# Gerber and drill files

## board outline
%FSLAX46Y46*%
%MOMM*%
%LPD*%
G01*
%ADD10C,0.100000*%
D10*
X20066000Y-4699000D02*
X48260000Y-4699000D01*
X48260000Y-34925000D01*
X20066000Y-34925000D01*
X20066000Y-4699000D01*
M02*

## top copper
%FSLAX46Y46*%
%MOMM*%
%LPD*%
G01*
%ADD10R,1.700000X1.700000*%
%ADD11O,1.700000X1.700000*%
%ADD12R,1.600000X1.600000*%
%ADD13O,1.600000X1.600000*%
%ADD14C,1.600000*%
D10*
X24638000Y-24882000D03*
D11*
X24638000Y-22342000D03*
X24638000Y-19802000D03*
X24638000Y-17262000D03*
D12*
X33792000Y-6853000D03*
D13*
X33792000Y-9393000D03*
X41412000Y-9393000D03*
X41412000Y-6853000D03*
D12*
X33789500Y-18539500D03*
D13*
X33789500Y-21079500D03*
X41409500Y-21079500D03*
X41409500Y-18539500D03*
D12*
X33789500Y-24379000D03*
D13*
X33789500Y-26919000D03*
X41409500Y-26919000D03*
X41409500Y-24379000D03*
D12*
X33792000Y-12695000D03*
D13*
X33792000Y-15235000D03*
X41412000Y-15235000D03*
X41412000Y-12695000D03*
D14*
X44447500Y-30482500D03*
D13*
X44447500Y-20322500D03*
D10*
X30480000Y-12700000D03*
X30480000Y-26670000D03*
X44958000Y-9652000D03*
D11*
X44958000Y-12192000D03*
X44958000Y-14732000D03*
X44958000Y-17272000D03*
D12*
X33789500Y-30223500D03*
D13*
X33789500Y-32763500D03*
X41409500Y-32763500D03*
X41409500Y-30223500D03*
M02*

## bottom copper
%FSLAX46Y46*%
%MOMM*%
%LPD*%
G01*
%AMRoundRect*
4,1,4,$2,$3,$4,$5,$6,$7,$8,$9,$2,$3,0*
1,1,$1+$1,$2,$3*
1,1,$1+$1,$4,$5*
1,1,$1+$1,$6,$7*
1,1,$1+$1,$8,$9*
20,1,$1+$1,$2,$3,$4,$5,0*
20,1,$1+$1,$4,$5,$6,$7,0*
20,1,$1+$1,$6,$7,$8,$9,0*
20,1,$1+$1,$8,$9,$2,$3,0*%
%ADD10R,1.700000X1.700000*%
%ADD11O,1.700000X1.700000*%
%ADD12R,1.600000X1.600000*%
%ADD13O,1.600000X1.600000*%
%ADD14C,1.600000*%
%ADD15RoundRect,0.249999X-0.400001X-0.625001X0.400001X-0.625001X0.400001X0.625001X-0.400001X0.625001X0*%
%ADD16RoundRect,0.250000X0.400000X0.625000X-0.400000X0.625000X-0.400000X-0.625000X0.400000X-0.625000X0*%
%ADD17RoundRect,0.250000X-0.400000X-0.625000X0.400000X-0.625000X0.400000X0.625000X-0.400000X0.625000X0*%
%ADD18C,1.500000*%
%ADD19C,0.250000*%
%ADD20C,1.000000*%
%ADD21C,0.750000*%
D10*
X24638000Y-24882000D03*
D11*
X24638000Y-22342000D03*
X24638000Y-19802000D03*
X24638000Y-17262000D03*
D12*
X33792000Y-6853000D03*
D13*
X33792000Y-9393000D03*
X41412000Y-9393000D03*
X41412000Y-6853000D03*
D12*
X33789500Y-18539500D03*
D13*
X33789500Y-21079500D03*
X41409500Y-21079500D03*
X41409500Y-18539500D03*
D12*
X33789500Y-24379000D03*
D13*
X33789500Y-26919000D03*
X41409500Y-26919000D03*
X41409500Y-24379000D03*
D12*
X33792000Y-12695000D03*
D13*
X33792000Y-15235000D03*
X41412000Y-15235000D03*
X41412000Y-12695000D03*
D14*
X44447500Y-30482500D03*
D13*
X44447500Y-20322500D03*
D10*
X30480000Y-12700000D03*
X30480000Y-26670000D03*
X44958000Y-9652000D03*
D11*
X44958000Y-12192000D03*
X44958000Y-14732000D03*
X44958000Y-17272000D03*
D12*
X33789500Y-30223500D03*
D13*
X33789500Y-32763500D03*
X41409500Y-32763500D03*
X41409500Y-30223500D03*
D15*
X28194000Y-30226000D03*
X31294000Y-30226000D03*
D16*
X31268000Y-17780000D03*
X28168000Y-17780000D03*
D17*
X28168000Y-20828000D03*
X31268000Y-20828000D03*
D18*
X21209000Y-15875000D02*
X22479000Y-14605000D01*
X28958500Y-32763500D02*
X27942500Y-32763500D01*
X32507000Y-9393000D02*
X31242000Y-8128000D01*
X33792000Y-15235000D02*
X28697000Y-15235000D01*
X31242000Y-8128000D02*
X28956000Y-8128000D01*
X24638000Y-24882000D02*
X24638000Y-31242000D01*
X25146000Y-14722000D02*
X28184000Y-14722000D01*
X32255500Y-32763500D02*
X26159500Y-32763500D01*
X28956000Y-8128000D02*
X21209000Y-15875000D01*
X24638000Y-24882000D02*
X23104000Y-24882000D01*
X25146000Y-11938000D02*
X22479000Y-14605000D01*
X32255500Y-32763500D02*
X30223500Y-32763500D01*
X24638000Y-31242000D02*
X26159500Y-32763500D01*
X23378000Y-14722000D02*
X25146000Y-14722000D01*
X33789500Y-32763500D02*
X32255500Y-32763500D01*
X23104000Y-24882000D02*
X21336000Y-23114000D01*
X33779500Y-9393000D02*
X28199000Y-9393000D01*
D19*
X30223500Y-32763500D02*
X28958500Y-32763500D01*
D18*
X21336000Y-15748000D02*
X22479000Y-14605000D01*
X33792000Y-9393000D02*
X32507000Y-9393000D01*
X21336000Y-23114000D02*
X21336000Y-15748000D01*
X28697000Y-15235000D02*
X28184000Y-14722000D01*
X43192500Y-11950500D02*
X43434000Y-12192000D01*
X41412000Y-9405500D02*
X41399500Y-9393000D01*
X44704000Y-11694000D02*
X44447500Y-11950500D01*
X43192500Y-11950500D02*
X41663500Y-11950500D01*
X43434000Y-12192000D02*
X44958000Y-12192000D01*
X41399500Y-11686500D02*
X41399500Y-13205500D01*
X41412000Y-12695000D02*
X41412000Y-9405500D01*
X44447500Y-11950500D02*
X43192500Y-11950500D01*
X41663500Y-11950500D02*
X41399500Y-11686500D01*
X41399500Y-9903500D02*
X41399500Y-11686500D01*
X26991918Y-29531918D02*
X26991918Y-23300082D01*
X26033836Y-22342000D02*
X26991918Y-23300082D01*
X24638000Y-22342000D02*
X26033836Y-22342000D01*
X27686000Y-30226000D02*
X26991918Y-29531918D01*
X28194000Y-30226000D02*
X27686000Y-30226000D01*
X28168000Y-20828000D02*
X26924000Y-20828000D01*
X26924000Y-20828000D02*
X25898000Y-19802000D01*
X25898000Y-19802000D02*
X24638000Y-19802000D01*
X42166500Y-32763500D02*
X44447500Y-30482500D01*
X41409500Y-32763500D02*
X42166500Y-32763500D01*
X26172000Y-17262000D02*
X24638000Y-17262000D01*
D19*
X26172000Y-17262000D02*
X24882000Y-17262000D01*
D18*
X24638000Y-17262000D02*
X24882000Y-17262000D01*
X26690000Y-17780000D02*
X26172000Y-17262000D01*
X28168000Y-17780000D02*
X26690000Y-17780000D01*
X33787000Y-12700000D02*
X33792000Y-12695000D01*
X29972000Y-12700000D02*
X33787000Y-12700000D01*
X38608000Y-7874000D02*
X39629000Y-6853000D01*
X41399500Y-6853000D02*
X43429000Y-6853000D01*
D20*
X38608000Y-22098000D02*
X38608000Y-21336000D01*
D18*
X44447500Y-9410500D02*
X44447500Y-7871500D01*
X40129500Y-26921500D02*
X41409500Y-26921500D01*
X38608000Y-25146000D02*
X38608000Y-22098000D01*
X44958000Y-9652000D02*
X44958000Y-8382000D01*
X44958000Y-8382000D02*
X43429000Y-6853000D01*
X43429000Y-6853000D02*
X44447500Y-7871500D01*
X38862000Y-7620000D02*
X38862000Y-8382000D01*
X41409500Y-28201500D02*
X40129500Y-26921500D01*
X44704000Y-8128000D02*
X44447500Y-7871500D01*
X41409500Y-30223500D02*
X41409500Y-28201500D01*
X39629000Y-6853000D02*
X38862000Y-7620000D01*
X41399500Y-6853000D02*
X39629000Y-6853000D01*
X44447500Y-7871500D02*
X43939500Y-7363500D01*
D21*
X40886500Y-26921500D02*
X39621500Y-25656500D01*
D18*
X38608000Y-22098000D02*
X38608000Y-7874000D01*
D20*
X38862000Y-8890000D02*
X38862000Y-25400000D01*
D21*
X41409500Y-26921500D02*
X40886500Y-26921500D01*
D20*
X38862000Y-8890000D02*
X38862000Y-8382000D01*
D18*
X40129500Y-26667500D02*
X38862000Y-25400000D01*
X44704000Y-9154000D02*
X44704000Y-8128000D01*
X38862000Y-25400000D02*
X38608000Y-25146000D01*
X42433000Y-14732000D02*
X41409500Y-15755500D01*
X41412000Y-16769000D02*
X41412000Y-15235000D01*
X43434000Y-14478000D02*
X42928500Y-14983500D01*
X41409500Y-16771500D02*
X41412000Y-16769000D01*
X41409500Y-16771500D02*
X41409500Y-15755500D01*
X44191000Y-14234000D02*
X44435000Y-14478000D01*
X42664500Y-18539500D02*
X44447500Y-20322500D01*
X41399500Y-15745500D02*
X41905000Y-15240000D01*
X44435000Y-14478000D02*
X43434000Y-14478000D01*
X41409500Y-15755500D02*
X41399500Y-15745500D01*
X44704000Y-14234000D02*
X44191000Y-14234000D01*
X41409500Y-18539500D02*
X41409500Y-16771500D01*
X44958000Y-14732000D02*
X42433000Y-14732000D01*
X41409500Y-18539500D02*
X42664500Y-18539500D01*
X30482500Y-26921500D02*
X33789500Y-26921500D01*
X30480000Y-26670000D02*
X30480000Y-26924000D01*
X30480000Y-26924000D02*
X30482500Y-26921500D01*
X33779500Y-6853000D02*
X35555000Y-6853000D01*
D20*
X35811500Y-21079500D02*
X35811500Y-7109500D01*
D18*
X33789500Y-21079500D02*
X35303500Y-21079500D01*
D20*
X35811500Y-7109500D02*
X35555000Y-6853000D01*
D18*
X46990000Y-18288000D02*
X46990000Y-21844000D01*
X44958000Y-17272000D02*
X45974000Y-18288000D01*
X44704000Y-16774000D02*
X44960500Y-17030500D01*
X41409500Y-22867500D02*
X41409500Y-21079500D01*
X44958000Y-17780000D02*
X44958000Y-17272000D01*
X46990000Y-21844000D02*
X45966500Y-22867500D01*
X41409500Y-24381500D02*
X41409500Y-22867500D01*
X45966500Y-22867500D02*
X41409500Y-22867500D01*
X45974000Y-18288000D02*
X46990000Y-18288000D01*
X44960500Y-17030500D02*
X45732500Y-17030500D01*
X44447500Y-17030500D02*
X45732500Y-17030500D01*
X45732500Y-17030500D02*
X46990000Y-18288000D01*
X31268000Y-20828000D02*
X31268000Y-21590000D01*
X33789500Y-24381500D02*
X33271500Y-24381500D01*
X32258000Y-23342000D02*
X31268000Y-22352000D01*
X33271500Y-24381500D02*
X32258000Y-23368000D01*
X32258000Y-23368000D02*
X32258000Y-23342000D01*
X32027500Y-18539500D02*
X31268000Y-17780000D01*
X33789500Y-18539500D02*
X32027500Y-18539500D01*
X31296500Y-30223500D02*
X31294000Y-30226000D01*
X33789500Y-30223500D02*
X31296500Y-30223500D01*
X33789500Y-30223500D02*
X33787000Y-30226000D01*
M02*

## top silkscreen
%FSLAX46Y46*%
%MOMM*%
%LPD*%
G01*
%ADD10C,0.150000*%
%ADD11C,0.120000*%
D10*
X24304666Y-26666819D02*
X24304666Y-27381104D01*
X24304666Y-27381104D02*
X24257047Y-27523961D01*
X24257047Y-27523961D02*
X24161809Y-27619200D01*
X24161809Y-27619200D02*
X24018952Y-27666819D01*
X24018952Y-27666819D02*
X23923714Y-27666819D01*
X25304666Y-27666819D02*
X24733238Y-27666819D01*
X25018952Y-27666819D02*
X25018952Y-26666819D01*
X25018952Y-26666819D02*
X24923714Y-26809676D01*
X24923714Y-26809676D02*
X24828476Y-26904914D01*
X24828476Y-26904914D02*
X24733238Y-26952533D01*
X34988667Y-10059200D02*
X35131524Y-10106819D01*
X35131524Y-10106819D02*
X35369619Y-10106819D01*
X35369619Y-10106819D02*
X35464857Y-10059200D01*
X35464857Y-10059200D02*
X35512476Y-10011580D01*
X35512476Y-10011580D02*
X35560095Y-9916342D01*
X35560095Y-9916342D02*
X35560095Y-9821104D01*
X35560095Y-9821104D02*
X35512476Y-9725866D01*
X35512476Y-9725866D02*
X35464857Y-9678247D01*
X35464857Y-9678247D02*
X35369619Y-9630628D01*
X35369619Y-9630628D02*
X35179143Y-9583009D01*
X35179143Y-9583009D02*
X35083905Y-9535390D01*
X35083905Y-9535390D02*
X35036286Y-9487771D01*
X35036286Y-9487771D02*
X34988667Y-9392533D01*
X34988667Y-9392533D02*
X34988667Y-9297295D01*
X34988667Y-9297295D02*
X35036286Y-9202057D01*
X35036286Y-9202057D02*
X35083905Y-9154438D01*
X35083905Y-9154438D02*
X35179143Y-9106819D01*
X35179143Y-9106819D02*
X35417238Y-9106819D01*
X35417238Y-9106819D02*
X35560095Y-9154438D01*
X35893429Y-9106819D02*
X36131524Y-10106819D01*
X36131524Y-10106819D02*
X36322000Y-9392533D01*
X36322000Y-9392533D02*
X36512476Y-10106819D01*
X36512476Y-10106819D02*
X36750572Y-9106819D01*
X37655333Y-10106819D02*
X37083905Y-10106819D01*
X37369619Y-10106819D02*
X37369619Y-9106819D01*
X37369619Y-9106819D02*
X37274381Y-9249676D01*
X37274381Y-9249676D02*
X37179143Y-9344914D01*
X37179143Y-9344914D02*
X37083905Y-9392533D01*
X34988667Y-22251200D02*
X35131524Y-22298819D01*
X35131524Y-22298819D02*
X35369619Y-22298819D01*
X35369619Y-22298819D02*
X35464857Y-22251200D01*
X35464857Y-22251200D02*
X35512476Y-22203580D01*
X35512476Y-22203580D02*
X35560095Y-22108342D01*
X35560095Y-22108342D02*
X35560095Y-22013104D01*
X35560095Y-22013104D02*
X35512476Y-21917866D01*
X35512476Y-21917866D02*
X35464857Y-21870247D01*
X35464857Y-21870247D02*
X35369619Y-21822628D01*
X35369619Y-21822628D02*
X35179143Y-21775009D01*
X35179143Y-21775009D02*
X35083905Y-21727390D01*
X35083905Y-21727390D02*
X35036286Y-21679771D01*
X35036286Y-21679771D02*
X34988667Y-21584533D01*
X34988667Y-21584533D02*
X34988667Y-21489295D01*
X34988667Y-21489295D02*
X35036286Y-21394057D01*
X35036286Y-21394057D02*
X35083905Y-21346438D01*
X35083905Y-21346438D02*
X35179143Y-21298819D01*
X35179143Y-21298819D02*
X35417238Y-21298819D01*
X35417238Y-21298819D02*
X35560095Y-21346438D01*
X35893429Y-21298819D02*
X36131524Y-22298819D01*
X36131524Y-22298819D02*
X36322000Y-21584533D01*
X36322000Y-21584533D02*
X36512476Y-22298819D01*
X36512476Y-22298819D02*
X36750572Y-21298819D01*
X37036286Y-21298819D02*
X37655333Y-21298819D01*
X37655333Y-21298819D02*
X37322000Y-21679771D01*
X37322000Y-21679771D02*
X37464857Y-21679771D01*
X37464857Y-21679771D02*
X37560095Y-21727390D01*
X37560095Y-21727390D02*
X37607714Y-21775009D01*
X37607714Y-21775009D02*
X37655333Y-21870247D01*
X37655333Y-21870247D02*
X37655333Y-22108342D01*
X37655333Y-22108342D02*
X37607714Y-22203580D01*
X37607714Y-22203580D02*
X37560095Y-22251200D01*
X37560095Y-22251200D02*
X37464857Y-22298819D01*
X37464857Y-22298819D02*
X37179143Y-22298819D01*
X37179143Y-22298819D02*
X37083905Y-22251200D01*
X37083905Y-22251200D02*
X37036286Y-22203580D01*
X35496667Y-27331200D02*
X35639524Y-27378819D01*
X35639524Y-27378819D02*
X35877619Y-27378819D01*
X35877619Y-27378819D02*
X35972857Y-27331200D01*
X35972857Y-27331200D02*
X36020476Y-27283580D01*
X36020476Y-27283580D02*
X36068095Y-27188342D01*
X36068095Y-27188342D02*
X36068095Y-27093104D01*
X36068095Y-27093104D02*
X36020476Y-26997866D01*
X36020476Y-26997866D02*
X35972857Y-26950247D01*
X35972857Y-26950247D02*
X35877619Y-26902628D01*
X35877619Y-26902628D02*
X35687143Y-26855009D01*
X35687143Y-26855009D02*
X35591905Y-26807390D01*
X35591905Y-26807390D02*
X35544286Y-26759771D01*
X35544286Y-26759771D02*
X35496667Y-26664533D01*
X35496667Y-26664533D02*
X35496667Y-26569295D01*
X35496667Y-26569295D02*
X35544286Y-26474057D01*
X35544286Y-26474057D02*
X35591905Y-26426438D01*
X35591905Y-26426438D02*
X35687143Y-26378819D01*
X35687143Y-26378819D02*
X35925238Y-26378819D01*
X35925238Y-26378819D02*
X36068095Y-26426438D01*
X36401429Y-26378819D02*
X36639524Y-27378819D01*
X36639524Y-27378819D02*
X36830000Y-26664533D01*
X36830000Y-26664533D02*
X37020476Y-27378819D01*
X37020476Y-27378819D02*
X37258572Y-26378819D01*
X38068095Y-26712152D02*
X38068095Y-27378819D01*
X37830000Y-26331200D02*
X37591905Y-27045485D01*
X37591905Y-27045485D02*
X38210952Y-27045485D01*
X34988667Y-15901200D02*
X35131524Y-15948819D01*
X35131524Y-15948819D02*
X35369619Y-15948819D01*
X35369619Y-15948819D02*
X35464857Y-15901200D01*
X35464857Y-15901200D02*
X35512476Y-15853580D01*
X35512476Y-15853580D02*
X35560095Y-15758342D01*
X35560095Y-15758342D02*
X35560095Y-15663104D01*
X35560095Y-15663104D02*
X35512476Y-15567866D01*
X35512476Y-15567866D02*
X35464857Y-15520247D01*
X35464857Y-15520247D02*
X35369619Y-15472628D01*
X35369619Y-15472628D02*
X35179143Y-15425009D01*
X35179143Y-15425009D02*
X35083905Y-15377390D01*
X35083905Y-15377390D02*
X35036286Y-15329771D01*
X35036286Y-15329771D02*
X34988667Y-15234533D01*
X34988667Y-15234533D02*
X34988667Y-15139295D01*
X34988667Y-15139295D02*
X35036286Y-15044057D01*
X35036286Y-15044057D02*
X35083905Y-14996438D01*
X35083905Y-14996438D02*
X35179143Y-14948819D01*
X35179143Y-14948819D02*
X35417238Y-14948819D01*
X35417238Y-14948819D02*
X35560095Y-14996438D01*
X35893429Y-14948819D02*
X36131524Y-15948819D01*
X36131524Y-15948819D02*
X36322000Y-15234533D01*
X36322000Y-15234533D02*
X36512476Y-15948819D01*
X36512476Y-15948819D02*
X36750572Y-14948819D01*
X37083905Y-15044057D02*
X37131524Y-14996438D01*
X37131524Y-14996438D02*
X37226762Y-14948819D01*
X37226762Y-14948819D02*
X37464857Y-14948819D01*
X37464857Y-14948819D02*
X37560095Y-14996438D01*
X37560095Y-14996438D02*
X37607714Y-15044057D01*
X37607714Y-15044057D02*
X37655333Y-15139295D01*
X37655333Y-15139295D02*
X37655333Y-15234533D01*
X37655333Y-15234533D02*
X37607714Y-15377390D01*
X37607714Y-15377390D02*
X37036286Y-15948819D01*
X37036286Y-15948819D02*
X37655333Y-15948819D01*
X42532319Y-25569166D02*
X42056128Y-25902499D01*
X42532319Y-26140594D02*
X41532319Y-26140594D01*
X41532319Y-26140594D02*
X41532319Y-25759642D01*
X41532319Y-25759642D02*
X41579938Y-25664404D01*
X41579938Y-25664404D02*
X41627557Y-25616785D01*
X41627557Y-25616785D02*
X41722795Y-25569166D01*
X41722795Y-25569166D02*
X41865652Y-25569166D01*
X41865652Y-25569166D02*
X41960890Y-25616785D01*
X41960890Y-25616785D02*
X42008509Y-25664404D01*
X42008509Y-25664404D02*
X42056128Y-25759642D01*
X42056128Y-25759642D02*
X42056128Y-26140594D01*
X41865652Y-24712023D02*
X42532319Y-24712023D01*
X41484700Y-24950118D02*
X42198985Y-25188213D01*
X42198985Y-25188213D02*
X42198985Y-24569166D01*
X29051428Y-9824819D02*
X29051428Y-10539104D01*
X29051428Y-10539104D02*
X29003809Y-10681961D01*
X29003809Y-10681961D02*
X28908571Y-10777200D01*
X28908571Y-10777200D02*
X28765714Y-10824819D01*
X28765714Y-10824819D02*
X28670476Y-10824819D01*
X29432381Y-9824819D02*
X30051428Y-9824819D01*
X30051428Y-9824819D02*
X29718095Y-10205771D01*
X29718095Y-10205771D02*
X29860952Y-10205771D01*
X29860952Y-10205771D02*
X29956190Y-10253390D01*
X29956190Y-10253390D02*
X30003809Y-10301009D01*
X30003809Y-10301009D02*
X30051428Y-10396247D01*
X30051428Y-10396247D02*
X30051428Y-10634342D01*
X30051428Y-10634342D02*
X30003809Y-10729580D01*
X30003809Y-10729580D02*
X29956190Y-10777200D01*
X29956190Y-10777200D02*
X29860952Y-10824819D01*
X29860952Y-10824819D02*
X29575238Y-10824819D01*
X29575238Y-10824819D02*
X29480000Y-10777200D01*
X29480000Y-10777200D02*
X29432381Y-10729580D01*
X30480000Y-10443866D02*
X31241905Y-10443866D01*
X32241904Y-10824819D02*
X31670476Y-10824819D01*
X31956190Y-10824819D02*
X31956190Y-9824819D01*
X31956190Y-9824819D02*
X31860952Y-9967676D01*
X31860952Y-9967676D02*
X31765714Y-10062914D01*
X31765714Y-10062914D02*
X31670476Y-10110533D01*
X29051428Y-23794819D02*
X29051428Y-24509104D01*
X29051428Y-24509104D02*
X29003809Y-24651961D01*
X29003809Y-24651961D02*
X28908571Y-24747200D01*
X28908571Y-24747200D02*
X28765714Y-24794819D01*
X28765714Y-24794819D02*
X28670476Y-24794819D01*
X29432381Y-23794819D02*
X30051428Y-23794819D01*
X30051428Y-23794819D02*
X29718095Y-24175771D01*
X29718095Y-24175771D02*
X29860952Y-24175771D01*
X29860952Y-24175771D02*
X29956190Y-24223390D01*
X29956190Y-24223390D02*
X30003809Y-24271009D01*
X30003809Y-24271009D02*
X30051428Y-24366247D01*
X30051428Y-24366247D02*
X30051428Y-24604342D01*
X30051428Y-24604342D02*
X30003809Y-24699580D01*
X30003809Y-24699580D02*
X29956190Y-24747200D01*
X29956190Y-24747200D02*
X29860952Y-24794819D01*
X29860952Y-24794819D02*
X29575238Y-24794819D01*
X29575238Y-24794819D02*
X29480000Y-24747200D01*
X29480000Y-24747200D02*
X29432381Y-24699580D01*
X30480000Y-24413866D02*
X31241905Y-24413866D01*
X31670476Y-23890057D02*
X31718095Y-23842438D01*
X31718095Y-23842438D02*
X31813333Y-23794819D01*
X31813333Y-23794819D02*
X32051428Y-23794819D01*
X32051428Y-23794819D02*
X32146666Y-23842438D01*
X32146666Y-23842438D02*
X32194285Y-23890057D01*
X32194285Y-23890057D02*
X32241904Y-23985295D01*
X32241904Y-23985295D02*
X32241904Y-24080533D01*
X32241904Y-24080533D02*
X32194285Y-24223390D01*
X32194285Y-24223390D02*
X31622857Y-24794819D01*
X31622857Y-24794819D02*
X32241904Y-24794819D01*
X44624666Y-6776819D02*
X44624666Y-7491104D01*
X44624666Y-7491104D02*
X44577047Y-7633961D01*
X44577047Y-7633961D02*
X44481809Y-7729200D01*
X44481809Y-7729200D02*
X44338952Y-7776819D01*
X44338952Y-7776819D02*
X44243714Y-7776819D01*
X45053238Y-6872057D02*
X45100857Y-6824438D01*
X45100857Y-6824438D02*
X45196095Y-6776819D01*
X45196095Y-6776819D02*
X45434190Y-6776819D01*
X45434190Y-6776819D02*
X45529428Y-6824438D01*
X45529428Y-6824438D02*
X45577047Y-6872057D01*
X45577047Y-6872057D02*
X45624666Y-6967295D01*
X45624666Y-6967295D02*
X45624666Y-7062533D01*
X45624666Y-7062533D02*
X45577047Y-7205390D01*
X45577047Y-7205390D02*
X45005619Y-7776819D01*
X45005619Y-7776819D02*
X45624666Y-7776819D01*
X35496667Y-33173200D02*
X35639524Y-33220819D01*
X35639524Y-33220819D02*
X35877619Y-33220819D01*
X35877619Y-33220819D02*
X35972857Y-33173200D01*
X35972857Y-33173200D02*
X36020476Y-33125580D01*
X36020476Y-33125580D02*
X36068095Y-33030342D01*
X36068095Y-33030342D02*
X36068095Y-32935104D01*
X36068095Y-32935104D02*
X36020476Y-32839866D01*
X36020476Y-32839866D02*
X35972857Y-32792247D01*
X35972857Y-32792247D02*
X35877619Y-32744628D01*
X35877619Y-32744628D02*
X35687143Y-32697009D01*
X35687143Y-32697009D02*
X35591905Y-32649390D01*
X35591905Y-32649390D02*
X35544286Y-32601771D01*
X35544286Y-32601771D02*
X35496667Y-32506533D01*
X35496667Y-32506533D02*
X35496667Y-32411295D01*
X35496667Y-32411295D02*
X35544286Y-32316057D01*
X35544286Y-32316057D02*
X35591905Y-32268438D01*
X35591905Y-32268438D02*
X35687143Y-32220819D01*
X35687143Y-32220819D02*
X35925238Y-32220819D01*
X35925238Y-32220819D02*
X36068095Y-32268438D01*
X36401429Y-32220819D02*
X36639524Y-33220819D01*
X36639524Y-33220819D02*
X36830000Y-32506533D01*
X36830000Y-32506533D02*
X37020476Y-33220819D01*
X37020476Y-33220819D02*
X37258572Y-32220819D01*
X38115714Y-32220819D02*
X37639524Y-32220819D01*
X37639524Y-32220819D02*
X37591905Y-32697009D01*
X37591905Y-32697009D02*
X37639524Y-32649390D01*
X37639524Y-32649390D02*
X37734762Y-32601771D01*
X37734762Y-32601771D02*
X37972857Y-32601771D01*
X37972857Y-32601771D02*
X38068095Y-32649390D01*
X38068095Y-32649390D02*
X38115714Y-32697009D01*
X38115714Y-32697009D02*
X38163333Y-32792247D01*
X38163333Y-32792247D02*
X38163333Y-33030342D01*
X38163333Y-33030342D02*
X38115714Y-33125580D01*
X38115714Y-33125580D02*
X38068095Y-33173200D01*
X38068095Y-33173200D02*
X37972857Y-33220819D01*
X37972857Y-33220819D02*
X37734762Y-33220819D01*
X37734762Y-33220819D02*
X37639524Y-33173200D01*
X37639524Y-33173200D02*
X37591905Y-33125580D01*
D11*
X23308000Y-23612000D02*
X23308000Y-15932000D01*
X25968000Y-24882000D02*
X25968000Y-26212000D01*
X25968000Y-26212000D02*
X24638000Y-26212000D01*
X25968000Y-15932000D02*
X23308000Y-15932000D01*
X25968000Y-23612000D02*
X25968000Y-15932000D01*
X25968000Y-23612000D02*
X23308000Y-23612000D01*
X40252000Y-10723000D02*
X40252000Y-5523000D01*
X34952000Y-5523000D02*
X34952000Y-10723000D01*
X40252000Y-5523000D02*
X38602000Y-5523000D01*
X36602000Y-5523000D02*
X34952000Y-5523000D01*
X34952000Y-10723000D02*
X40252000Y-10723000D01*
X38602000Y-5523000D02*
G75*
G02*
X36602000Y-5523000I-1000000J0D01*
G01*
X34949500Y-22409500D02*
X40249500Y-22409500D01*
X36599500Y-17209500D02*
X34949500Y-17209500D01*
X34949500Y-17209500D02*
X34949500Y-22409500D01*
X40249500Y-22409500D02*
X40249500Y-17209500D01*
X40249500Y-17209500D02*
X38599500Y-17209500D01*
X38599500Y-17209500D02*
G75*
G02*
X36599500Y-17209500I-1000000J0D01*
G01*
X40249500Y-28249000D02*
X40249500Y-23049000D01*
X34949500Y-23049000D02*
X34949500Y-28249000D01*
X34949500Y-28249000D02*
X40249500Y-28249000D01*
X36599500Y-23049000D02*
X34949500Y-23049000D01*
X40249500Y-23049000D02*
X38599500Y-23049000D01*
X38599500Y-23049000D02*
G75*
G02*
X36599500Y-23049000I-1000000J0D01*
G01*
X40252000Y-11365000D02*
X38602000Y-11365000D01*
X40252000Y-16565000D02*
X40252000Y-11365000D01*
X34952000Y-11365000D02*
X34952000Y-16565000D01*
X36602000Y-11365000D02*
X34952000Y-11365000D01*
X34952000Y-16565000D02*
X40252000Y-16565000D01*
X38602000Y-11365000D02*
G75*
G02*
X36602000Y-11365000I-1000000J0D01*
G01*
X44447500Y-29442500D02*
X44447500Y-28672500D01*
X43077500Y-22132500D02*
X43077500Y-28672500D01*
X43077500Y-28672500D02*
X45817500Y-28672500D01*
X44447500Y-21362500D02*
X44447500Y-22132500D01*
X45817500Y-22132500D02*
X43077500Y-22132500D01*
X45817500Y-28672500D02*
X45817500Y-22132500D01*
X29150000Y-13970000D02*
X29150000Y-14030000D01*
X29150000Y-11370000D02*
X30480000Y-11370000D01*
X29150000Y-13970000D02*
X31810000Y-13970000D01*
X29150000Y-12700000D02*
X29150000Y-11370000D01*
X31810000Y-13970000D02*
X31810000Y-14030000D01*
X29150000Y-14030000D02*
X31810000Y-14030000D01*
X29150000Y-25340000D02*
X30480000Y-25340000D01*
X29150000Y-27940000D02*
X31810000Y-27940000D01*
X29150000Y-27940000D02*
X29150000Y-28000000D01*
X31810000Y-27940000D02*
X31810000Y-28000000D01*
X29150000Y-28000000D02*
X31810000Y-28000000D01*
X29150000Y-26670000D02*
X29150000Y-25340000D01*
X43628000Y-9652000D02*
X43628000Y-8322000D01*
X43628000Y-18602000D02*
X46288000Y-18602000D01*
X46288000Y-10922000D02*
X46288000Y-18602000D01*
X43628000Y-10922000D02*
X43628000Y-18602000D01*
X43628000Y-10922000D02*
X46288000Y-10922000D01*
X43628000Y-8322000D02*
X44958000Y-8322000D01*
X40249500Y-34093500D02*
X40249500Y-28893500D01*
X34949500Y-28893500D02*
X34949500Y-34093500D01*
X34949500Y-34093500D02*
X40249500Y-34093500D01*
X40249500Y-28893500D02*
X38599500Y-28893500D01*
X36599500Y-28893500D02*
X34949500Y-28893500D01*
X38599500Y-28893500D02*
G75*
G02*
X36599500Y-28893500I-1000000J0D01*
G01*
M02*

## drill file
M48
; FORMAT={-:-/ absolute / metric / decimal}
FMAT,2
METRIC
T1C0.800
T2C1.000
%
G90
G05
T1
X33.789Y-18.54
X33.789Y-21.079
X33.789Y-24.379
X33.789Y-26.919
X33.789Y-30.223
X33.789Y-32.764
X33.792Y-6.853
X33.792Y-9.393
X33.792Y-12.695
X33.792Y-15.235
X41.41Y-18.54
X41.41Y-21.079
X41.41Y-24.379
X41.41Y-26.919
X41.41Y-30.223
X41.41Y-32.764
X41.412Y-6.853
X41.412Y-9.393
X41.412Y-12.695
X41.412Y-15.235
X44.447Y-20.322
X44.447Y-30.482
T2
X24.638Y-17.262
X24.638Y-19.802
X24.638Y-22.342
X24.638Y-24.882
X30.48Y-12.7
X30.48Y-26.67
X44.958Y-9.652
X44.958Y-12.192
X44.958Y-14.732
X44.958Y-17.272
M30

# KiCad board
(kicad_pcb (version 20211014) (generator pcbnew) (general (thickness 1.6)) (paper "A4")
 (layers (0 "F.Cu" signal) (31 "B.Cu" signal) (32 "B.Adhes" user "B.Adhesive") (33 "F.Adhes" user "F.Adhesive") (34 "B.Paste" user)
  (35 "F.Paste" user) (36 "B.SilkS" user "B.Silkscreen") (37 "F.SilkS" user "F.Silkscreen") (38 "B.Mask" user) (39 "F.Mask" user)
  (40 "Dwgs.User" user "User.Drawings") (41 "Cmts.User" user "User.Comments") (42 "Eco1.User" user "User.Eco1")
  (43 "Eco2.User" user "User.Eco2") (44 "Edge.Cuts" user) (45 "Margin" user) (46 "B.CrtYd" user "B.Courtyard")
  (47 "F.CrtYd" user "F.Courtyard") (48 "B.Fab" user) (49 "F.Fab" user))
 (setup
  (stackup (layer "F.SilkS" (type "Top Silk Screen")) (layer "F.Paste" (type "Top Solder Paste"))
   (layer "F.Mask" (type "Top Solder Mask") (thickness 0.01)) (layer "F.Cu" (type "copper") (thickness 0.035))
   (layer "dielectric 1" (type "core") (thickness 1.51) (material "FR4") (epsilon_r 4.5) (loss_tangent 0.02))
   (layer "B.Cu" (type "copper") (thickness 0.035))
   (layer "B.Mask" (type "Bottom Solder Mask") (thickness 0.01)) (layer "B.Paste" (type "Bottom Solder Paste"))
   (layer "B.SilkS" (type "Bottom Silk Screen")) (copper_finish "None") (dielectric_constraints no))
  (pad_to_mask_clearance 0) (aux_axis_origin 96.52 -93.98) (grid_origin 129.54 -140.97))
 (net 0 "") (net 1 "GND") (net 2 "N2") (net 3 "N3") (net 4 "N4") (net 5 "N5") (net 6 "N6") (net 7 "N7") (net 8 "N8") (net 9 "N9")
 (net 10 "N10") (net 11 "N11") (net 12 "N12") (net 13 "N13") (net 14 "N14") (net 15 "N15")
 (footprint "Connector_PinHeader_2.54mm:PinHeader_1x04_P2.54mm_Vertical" (layer "F.Cu") (at 24.638 24.882 180)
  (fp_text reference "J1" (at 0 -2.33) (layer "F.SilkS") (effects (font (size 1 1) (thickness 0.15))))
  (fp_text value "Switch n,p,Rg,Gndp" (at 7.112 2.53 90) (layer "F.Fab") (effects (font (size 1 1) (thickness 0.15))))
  (fp_line (start 1.33 1.27) (end 1.33 8.95) (layer "F.SilkS") (width 0.12))
  (fp_line (start -1.33 0) (end -1.33 -1.33) (layer "F.SilkS") (width 0.12))
  (fp_line (start -1.33 -1.33) (end 0 -1.33) (layer "F.SilkS") (width 0.12))
  (fp_line (start -1.33 8.95) (end 1.33 8.95) (layer "F.SilkS") (width 0.12))
  (fp_line (start -1.33 1.27) (end -1.33 8.95) (layer "F.SilkS") (width 0.12))
  (fp_line (start -1.33 1.27) (end 1.33 1.27) (layer "F.SilkS") (width 0.12))
  (pad "1" thru_hole rect (at 0 0 180) (size 1.7 1.7) (drill 1) (layers *.Cu *.Mask) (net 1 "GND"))
  (pad "2" thru_hole oval (at 0 2.54 180) (size 1.7 1.7) (drill 1) (layers *.Cu *.Mask) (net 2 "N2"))
  (pad "3" thru_hole oval (at 0 5.08 180) (size 1.7 1.7) (drill 1) (layers *.Cu *.Mask) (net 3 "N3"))
  (pad "4" thru_hole oval (at 0 7.62 180) (size 1.7 1.7) (drill 1) (layers *.Cu *.Mask) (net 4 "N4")))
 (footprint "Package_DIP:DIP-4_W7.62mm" (layer "F.Cu") (at 33.792 6.853)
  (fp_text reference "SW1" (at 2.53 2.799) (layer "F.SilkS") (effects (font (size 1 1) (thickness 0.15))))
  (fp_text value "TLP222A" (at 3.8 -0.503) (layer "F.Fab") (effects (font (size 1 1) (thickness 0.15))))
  (fp_line (start 6.46 3.87) (end 6.46 -1.33) (layer "F.SilkS") (width 0.12))
  (fp_line (start 1.16 -1.33) (end 1.16 3.87) (layer "F.SilkS") (width 0.12))
  (fp_line (start 6.46 -1.33) (end 4.81 -1.33) (layer "F.SilkS") (width 0.12))
  (fp_line (start 2.81 -1.33) (end 1.16 -1.33) (layer "F.SilkS") (width 0.12))
  (fp_line (start 1.16 3.87) (end 6.46 3.87) (layer "F.SilkS") (width 0.12))
  (fp_arc (start 4.81 -1.33) (mid 3.81 -0.33) (end 2.81 -1.33) (layer "F.SilkS") (width 0.12))
  (pad "1" thru_hole rect locked (at 0 0) (size 1.6 1.6) (drill 0.8) (layers *.Cu *.Mask) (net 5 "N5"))
  (pad "2" thru_hole oval locked (at 0 2.54) (size 1.6 1.6) (drill 0.8) (layers *.Cu *.Mask) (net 1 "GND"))
  (pad "3" thru_hole oval locked (at 7.62 2.54) (size 1.6 1.6) (drill 0.8) (layers *.Cu *.Mask) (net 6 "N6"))
  (pad "4" thru_hole oval locked (at 7.62 0) (size 1.6 1.6) (drill 0.8) (layers *.Cu *.Mask) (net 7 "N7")))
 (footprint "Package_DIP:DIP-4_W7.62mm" (layer "F.Cu") (at 33.7895 18.5395)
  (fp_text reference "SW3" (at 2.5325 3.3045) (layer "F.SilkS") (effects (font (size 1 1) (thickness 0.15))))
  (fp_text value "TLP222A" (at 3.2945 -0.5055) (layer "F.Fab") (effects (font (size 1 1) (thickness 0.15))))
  (fp_line (start 1.16 3.87) (end 6.46 3.87) (layer "F.SilkS") (width 0.12))
  (fp_line (start 2.81 -1.33) (end 1.16 -1.33) (layer "F.SilkS") (width 0.12))
  (fp_line (start 1.16 -1.33) (end 1.16 3.87) (layer "F.SilkS") (width 0.12))
  (fp_line (start 6.46 3.87) (end 6.46 -1.33) (layer "F.SilkS") (width 0.12))
  (fp_line (start 6.46 -1.33) (end 4.81 -1.33) (layer "F.SilkS") (width 0.12))
  (fp_arc (start 4.81 -1.33) (mid 3.81 -0.33) (end 2.81 -1.33) (layer "F.SilkS") (width 0.12))
  (pad "1" thru_hole rect locked (at 0 0) (size 1.6 1.6) (drill 0.8) (layers *.Cu *.Mask) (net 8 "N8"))
  (pad "2" thru_hole oval locked (at 0 2.54) (size 1.6 1.6) (drill 0.8) (layers *.Cu *.Mask) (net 5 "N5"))
  (pad "3" thru_hole oval locked (at 7.62 2.54) (size 1.6 1.6) (drill 0.8) (layers *.Cu *.Mask) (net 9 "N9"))
  (pad "4" thru_hole oval locked (at 7.62 0) (size 1.6 1.6) (drill 0.8) (layers *.Cu *.Mask) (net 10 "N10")))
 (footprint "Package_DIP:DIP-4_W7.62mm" (layer "F.Cu") (at 33.7895 24.379)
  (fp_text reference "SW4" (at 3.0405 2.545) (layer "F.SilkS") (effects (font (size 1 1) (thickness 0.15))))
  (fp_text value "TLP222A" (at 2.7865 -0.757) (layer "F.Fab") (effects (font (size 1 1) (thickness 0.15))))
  (fp_line (start 6.46 3.87) (end 6.46 -1.33) (layer "F.SilkS") (width 0.12))
  (fp_line (start 1.16 -1.33) (end 1.16 3.87) (layer "F.SilkS") (width 0.12))
  (fp_line (start 1.16 3.87) (end 6.46 3.87) (layer "F.SilkS") (width 0.12))
  (fp_line (start 2.81 -1.33) (end 1.16 -1.33) (layer "F.SilkS") (width 0.12))
  (fp_line (start 6.46 -1.33) (end 4.81 -1.33) (layer "F.SilkS") (width 0.12))
  (fp_arc (start 4.81 -1.33) (mid 3.81 -0.33) (end 2.81 -1.33) (layer "F.SilkS") (width 0.12))
  (pad "1" thru_hole rect locked (at 0 0) (size 1.6 1.6) (drill 0.8) (layers *.Cu *.Mask) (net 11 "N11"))
  (pad "2" thru_hole oval locked (at 0 2.54) (size 1.6 1.6) (drill 0.8) (layers *.Cu *.Mask) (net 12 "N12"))
  (pad "3" thru_hole oval locked (at 7.62 2.54) (size 1.6 1.6) (drill 0.8) (layers *.Cu *.Mask) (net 7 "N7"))
  (pad "4" thru_hole oval locked (at 7.62 0) (size 1.6 1.6) (drill 0.8) (layers *.Cu *.Mask) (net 9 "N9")))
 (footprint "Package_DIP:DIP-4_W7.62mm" (layer "F.Cu") (at 33.792 12.695)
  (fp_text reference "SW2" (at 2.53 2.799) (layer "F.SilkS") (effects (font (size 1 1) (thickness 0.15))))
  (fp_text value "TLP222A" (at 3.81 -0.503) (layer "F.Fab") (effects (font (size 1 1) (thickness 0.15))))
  (fp_line (start 6.46 -1.33) (end 4.81 -1.33) (layer "F.SilkS") (width 0.12))
  (fp_line (start 6.46 3.87) (end 6.46 -1.33) (layer "F.SilkS") (width 0.12))
  (fp_line (start 1.16 -1.33) (end 1.16 3.87) (layer "F.SilkS") (width 0.12))
  (fp_line (start 2.81 -1.33) (end 1.16 -1.33) (layer "F.SilkS") (width 0.12))
  (fp_line (start 1.16 3.87) (end 6.46 3.87) (layer "F.SilkS") (width 0.12))
  (fp_arc (start 4.81 -1.33) (mid 3.81 -0.33) (end 2.81 -1.33) (layer "F.SilkS") (width 0.12))
  (pad "1" thru_hole rect locked (at 0 0) (size 1.6 1.6) (drill 0.8) (layers *.Cu *.Mask) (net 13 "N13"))
  (pad "2" thru_hole oval locked (at 0 2.54) (size 1.6 1.6) (drill 0.8) (layers *.Cu *.Mask) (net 1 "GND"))
  (pad "3" thru_hole oval locked (at 7.62 2.54) (size 1.6 1.6) (drill 0.8) (layers *.Cu *.Mask) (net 10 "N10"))
  (pad "4" thru_hole oval locked (at 7.62 0) (size 1.6 1.6) (drill 0.8) (layers *.Cu *.Mask) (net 6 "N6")))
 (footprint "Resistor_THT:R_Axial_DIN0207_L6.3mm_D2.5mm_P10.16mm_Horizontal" (layer "F.Cu") (at 44.4475 30.4825 90)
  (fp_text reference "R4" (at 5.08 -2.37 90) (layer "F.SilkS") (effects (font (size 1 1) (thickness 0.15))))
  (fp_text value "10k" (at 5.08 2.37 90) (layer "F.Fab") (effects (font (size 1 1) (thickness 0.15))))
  (fp_line (start 1.04 0) (end 1.81 0) (layer "F.SilkS") (width 0.12))
  (fp_line (start 8.35 -1.37) (end 1.81 -1.37) (layer "F.SilkS") (width 0.12))
  (fp_line (start 1.81 -1.37) (end 1.81 1.37) (layer "F.SilkS") (width 0.12))
  (fp_line (start 9.12 0) (end 8.35 0) (layer "F.SilkS") (width 0.12))
  (fp_line (start 8.35 1.37) (end 8.35 -1.37) (layer "F.SilkS") (width 0.12))
  (fp_line (start 1.81 1.37) (end 8.35 1.37) (layer "F.SilkS") (width 0.12))
  (pad "1" thru_hole circle locked (at 0 0 90) (size 1.6 1.6) (drill 0.8) (layers *.Cu *.Mask) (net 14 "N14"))
  (pad "2" thru_hole oval locked (at 10.16 0 90) (size 1.6 1.6) (drill 0.8) (layers *.Cu *.Mask) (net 10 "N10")))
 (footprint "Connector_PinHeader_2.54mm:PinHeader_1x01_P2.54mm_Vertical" (layer "F.Cu") (at 30.48 12.7)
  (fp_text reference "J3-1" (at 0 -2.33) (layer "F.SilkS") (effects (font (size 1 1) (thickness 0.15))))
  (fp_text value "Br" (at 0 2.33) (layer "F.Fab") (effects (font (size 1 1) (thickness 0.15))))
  (fp_line (start -1.33 1.27) (end -1.33 1.33) (layer "F.SilkS") (width 0.12))
  (fp_line (start -1.33 -1.33) (end 0 -1.33) (layer "F.SilkS") (width 0.12))
  (fp_line (start -1.33 1.27) (end 1.33 1.27) (layer "F.SilkS") (width 0.12))
  (fp_line (start -1.33 0) (end -1.33 -1.33) (layer "F.SilkS") (width 0.12))
  (fp_line (start 1.33 1.27) (end 1.33 1.33) (layer "F.SilkS") (width 0.12))
  (fp_line (start -1.33 1.33) (end 1.33 1.33) (layer "F.SilkS") (width 0.12))
  (pad "1" thru_hole rect (at 0 0) (size 1.7 1.7) (drill 1) (layers *.Cu *.Mask) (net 13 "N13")))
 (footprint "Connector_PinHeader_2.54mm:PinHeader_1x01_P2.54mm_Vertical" (layer "F.Cu") (at 30.48 26.67)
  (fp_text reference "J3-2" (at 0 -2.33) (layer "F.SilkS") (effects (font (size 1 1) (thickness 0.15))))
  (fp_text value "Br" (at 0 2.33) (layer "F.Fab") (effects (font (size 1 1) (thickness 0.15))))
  (fp_line (start -1.33 -1.33) (end 0 -1.33) (layer "F.SilkS") (width 0.12))
  (fp_line (start -1.33 1.27) (end 1.33 1.27) (layer "F.SilkS") (width 0.12))
  (fp_line (start -1.33 1.27) (end -1.33 1.33) (layer "F.SilkS") (width 0.12))
  (fp_line (start 1.33 1.27) (end 1.33 1.33) (layer "F.SilkS") (width 0.12))
  (fp_line (start -1.33 1.33) (end 1.33 1.33) (layer "F.SilkS") (width 0.12))
  (fp_line (start -1.33 0) (end -1.33 -1.33) (layer "F.SilkS") (width 0.12))
  (pad "1" thru_hole rect (at 0 0) (size 1.7 1.7) (drill 1) (layers *.Cu *.Mask) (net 12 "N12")))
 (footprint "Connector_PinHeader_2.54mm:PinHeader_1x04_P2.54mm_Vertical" (layer "F.Cu") (at 44.958 9.652)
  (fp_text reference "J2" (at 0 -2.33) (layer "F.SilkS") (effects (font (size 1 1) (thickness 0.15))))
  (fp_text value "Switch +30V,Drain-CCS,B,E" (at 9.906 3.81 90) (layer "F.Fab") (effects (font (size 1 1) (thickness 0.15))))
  (fp_line (start -1.33 0) (end -1.33 -1.33) (layer "F.SilkS") (width 0.12))
  (fp_line (start -1.33 8.95) (end 1.33 8.95) (layer "F.SilkS") (width 0.12))
  (fp_line (start 1.33 1.27) (end 1.33 8.95) (layer "F.SilkS") (width 0.12))
  (fp_line (start -1.33 1.27) (end -1.33 8.95) (layer "F.SilkS") (width 0.12))
  (fp_line (start -1.33 1.27) (end 1.33 1.27) (layer "F.SilkS") (width 0.12))
  (fp_line (start -1.33 -1.33) (end 0 -1.33) (layer "F.SilkS") (width 0.12))
  (pad "1" thru_hole rect (at 0 0) (size 1.7 1.7) (drill 1) (layers *.Cu *.Mask) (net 7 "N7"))
  (pad "2" thru_hole oval (at 0 2.54) (size 1.7 1.7) (drill 1) (layers *.Cu *.Mask) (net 6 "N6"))
  (pad "3" thru_hole oval (at 0 5.08) (size 1.7 1.7) (drill 1) (layers *.Cu *.Mask) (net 10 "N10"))
  (pad "4" thru_hole oval (at 0 7.62) (size 1.7 1.7) (drill 1) (layers *.Cu *.Mask) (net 9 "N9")))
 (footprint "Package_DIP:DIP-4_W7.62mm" (layer "F.Cu") (at 33.7895 30.2235)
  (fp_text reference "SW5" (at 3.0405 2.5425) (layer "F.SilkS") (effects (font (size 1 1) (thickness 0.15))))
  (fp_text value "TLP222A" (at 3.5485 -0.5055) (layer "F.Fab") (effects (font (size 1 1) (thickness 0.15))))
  (fp_line (start 6.46 3.87) (end 6.46 -1.33) (layer "F.SilkS") (width 0.12))
  (fp_line (start 1.16 -1.33) (end 1.16 3.87) (layer "F.SilkS") (width 0.12))
  (fp_line (start 1.16 3.87) (end 6.46 3.87) (layer "F.SilkS") (width 0.12))
  (fp_line (start 6.46 -1.33) (end 4.81 -1.33) (layer "F.SilkS") (width 0.12))
  (fp_line (start 2.81 -1.33) (end 1.16 -1.33) (layer "F.SilkS") (width 0.12))
  (fp_arc (start 4.81 -1.33) (mid 3.81 -0.33) (end 2.81 -1.33) (layer "F.SilkS") (width 0.12))
  (pad "1" thru_hole rect (at 0 0) (size 1.6 1.6) (drill 0.8) (layers *.Cu *.Mask) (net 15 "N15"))
  (pad "2" thru_hole oval (at 0 2.54) (size 1.6 1.6) (drill 0.8) (layers *.Cu *.Mask) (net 1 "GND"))
  (pad "3" thru_hole oval (at 7.62 2.54) (size 1.6 1.6) (drill 0.8) (layers *.Cu *.Mask) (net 14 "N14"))
  (pad "4" thru_hole oval (at 7.62 0) (size 1.6 1.6) (drill 0.8) (layers *.Cu *.Mask) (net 7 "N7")))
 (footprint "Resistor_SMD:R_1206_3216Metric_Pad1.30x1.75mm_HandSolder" (layer "B.Cu") (at 29.744 30.226)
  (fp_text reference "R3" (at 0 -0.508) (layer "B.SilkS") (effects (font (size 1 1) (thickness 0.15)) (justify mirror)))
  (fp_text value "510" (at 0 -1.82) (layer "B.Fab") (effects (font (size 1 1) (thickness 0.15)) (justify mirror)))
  (pad "1" smd roundrect locked (at -1.55 0) (size 1.3 1.75) (layers "B.Cu" "B.Paste" "B.Mask") (roundrect_rratio 0.1923069231) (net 2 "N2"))
  (pad "2" smd roundrect locked (at 1.55 0) (size 1.3 1.75) (layers "B.Cu" "B.Paste" "B.Mask") (roundrect_rratio 0.1923069231)
   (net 15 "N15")))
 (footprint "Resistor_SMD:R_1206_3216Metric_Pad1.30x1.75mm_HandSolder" (layer "B.Cu") (at 29.718 17.78 180)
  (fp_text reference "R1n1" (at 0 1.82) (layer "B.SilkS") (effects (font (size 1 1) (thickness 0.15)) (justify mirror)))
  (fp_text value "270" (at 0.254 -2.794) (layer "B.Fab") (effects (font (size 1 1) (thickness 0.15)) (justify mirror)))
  (pad "1" smd roundrect (at -1.55 0 180) (size 1.3 1.75) (layers "B.Cu" "B.Paste" "B.Mask") (roundrect_rratio 0.192308) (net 8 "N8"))
  (pad "2" smd roundrect (at 1.55 0 180) (size 1.3 1.75) (layers "B.Cu" "B.Paste" "B.Mask") (roundrect_rratio 0.192308) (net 4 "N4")))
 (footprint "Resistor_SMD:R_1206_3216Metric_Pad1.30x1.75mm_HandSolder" (layer "B.Cu") (at 29.718 20.828)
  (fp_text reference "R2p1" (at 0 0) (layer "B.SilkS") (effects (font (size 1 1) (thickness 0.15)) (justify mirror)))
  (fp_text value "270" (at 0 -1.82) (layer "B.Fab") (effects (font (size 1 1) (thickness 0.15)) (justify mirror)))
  (pad "1" smd roundrect (at -1.55 0) (size 1.3 1.75) (layers "B.Cu" "B.Paste" "B.Mask") (roundrect_rratio 0.192308) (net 3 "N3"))
  (pad "2" smd roundrect (at 1.55 0) (size 1.3 1.75) (layers "B.Cu" "B.Paste" "B.Mask") (roundrect_rratio 0.192308) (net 11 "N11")))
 (gr_rect (start 20.066 4.699) (end 48.26 34.925) (layer "Edge.Cuts") (width 0.1) (fill none))
 (segment (start 21.209 15.875) (end 22.479 14.605) (width 1.5) (layer "B.Cu") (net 1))
 (segment (start 28.9585 32.7635) (end 27.9425 32.7635) (width 1.5) (layer "B.Cu") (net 1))
 (segment (start 32.507 9.393) (end 31.242 8.128) (width 1.5) (layer "B.Cu") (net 1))
 (segment (start 33.792 15.235) (end 28.697 15.235) (width 1.5) (layer "B.Cu") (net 1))
 (segment (start 31.242 8.128) (end 28.956 8.128) (width 1.5) (layer "B.Cu") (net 1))
 (segment (start 24.638 24.882) (end 24.638 31.242) (width 1.5) (layer "B.Cu") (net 1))
 (segment (start 25.146 14.722) (end 28.184 14.722) (width 1.5) (layer "B.Cu") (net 1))
 (segment (start 32.2555 32.7635) (end 26.1595 32.7635) (width 1.5) (layer "B.Cu") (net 1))
 (segment (start 28.956 8.128) (end 21.209 15.875) (width 1.5) (layer "B.Cu") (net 1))
 (segment (start 24.638 24.882) (end 23.104 24.882) (width 1.5) (layer "B.Cu") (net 1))
 (segment (start 25.146 11.938) (end 22.479 14.605) (width 1.5) (layer "B.Cu") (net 1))
 (segment (start 32.2555 32.7635) (end 30.2235 32.7635) (width 1.5) (layer "B.Cu") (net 1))
 (segment (start 24.638 31.242) (end 26.1595 32.7635) (width 1.5) (layer "B.Cu") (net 1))
 (segment (start 23.378 14.722) (end 25.146 14.722) (width 1.5) (layer "B.Cu") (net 1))
 (segment (start 33.7895 32.7635) (end 32.2555 32.7635) (width 1.5) (layer "B.Cu") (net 1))
 (segment (start 23.104 24.882) (end 21.336 23.114) (width 1.5) (layer "B.Cu") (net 1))
 (segment (start 33.7795 9.393) (end 28.199 9.393) (width 1.5) (layer "B.Cu") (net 1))
 (segment (start 30.2235 32.7635) (end 28.9585 32.7635) (width 0.25) (layer "B.Cu") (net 1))
 (segment (start 21.336 15.748) (end 22.479 14.605) (width 1.5) (layer "B.Cu") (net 1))
 (segment (start 33.792 9.393) (end 32.507 9.393) (width 1.5) (layer "B.Cu") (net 1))
 (segment (start 21.336 23.114) (end 21.336 15.748) (width 1.5) (layer "B.Cu") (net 1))
 (segment (start 28.697 15.235) (end 28.184 14.722) (width 1.5) (layer "B.Cu") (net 1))
 (segment (start 43.1925 11.9505) (end 43.434 12.192) (width 1.5) (layer "B.Cu") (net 6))
 (segment (start 41.412 9.4055) (end 41.3995 9.393) (width 1.5) (layer "B.Cu") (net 6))
 (segment (start 44.704 11.694) (end 44.4475 11.9505) (width 1.5) (layer "B.Cu") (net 6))
 (segment (start 43.1925 11.9505) (end 41.6635 11.9505) (width 1.5) (layer "B.Cu") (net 6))
 (segment (start 43.434 12.192) (end 44.958 12.192) (width 1.5) (layer "B.Cu") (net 6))
 (segment (start 41.3995 11.6865) (end 41.3995 13.2055) (width 1.5) (layer "B.Cu") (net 6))
 (segment (start 41.412 12.695) (end 41.412 9.4055) (width 1.5) (layer "B.Cu") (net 6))
 (segment (start 44.4475 11.9505) (end 43.1925 11.9505) (width 1.5) (layer "B.Cu") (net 6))
 (segment (start 41.6635 11.9505) (end 41.3995 11.6865) (width 1.5) (layer "B.Cu") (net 6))
 (segment (start 41.3995 9.9035) (end 41.3995 11.6865) (width 1.5) (layer "B.Cu") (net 6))
 (segment (start 26.991918 29.531918) (end 26.991918 23.300082) (width 1.5) (layer "B.Cu") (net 2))
 (segment (start 26.033836 22.342) (end 26.991918 23.300082) (width 1.5) (layer "B.Cu") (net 2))
 (segment (start 24.638 22.342) (end 26.033836 22.342) (width 1.5) (layer "B.Cu") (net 2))
 (segment (start 27.686 30.226) (end 26.991918 29.531918) (width 1.5) (layer "B.Cu") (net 2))
 (segment (start 28.194 30.226) (end 27.686 30.226) (width 1.5) (layer "B.Cu") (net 2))
 (segment (start 28.168 20.828) (end 26.924 20.828) (width 1.5) (layer "B.Cu") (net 3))
 (segment (start 26.924 20.828) (end 25.898 19.802) (width 1.5) (layer "B.Cu") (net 3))
 (segment (start 25.898 19.802) (end 24.638 19.802) (width 1.5) (layer "B.Cu") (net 3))
 (segment (start 42.1665 32.7635) (end 44.4475 30.4825) (width 1.5) (layer "B.Cu") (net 14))
 (segment (start 41.4095 32.7635) (end 42.1665 32.7635) (width 1.5) (layer "B.Cu") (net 14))
 (segment (start 26.172 17.262) (end 24.638 17.262) (width 1.5) (layer "B.Cu") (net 4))
 (segment (start 26.172 17.262) (end 24.882 17.262) (width 0.25) (layer "B.Cu") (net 4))
 (segment (start 24.638 17.262) (end 24.882 17.262) (width 1.5) (layer "B.Cu") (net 4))
 (segment (start 26.69 17.78) (end 26.172 17.262) (width 1.5) (layer "B.Cu") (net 4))
 (segment (start 28.168 17.78) (end 26.69 17.78) (width 1.5) (layer "B.Cu") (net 4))
 (segment (start 33.787 12.7) (end 33.792 12.695) (width 1.5) (layer "B.Cu") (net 13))
 (segment (start 29.972 12.7) (end 33.787 12.7) (width 1.5) (layer "B.Cu") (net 13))
 (segment (start 38.608 7.874) (end 39.629 6.853) (width 1.5) (layer "B.Cu") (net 7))
 (segment (start 41.3995 6.853) (end 43.429 6.853) (width 1.5) (layer "B.Cu") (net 7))
 (segment (start 38.608 22.098) (end 38.608 21.336) (width 1) (layer "B.Cu") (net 7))
 (segment (start 44.4475 9.4105) (end 44.4475 7.8715) (width 1.5) (layer "B.Cu") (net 7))
 (segment (start 40.1295 26.9215) (end 41.4095 26.9215) (width 1.5) (layer "B.Cu") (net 7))
 (segment (start 38.608 25.146) (end 38.608 22.098) (width 1.5) (layer "B.Cu") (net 7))
 (segment (start 44.958 9.652) (end 44.958 8.382) (width 1.5) (layer "B.Cu") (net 7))
 (segment (start 44.958 8.382) (end 43.429 6.853) (width 1.5) (layer "B.Cu") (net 7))
 (segment (start 43.429 6.853) (end 44.4475 7.8715) (width 1.5) (layer "B.Cu") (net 7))
 (segment (start 38.862 7.62) (end 38.862 8.382) (width 1.5) (layer "B.Cu") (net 7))
 (segment (start 41.4095 28.2015) (end 40.1295 26.9215) (width 1.5) (layer "B.Cu") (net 7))
 (segment (start 44.704 8.128) (end 44.4475 7.8715) (width 1.5) (layer "B.Cu") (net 7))
 (segment (start 41.4095 30.2235) (end 41.4095 28.2015) (width 1.5) (layer "B.Cu") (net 7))
 (segment (start 39.629 6.853) (end 38.862 7.62) (width 1.5) (layer "B.Cu") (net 7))
 (segment (start 41.3995 6.853) (end 39.629 6.853) (width 1.5) (layer "B.Cu") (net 7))
 (segment (start 44.4475 7.8715) (end 43.9395 7.3635) (width 1.5) (layer "B.Cu") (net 7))
 (segment (start 40.8865 26.9215) (end 39.6215 25.6565) (width 0.75) (layer "B.Cu") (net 7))
 (segment (start 38.608 22.098) (end 38.608 7.874) (width 1.5) (layer "B.Cu") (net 7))
 (segment (start 38.862 8.89) (end 38.862 25.4) (width 1) (layer "B.Cu") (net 7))
 (segment (start 41.4095 26.9215) (end 40.8865 26.9215) (width 0.75) (layer "B.Cu") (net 7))
 (segment (start 38.862 8.89) (end 38.862 8.382) (width 1) (layer "B.Cu") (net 7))
 (segment (start 40.1295 26.6675) (end 38.862 25.4) (width 1.5) (layer "B.Cu") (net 7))
 (segment (start 44.704 9.154) (end 44.704 8.128) (width 1.5) (layer "B.Cu") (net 7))
 (segment (start 38.862 25.4) (end 38.608 25.146) (width 1.5) (layer "B.Cu") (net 7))
 (segment (start 42.433 14.732) (end 41.4095 15.7555) (width 1.5) (layer "B.Cu") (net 10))
 (segment (start 41.412 16.769) (end 41.412 15.235) (width 1.5) (layer "B.Cu") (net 10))
 (segment (start 43.434 14.478) (end 42.9285 14.9835) (width 1.5) (layer "B.Cu") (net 10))
 (segment (start 41.4095 16.7715) (end 41.412 16.769) (width 1.5) (layer "B.Cu") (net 10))
 (segment (start 41.4095 16.7715) (end 41.4095 15.7555) (width 1.5) (layer "B.Cu") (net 10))
 (segment (start 44.191 14.234) (end 44.435 14.478) (width 1.5) (layer "B.Cu") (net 10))
 (segment (start 42.6645 18.5395) (end 44.4475 20.3225) (width 1.5) (layer "B.Cu") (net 10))
 (segment (start 41.3995 15.7455) (end 41.905 15.24) (width 1.5) (layer "B.Cu") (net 10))
 (segment (start 44.435 14.478) (end 43.434 14.478) (width 1.5) (layer "B.Cu") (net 10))
 (segment (start 41.4095 15.7555) (end 41.3995 15.7455) (width 1.5) (layer "B.Cu") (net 10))
 (segment (start 44.704 14.234) (end 44.191 14.234) (width 1.5) (layer "B.Cu") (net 10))
 (segment (start 41.4095 18.5395) (end 41.4095 16.7715) (width 1.5) (layer "B.Cu") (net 10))
 (segment (start 44.958 14.732) (end 42.433 14.732) (width 1.5) (layer "B.Cu") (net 10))
 (segment (start 41.4095 18.5395) (end 42.6645 18.5395) (width 1.5) (layer "B.Cu") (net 10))
 (segment (start 30.4825 26.9215) (end 33.7895 26.9215) (width 1.5) (layer "B.Cu") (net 12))
 (segment (start 30.48 26.67) (end 30.48 26.924) (width 1.5) (layer "B.Cu") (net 12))
 (segment (start 30.48 26.924) (end 30.4825 26.9215) (width 1.5) (layer "B.Cu") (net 12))
 (segment (start 33.7795 6.853) (end 35.555 6.853) (width 1.5) (layer "B.Cu") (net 5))
 (segment (start 35.8115 21.0795) (end 35.8115 7.1095) (width 1) (layer "B.Cu") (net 5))
 (segment (start 33.7895 21.0795) (end 35.3035 21.0795) (width 1.5) (layer "B.Cu") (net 5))
 (segment (start 35.8115 7.1095) (end 35.555 6.853) (width 1) (layer "B.Cu") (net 5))
 (segment (start 46.99 18.288) (end 46.99 21.844) (width 1.5) (layer "B.Cu") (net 9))
 (segment (start 44.958 17.272) (end 45.974 18.288) (width 1.5) (layer "B.Cu") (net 9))
 (segment (start 44.704 16.774) (end 44.9605 17.0305) (width 1.5) (layer "B.Cu") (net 9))
 (segment (start 41.4095 22.8675) (end 41.4095 21.0795) (width 1.5) (layer "B.Cu") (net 9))
 (segment (start 44.958 17.78) (end 44.958 17.272) (width 1.5) (layer "B.Cu") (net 9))
 (segment (start 46.99 21.844) (end 45.9665 22.8675) (width 1.5) (layer "B.Cu") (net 9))
 (segment (start 41.4095 24.3815) (end 41.4095 22.8675) (width 1.5) (layer "B.Cu") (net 9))
 (segment (start 45.9665 22.8675) (end 41.4095 22.8675) (width 1.5) (layer "B.Cu") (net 9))
 (segment (start 45.974 18.288) (end 46.99 18.288) (width 1.5) (layer "B.Cu") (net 9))
 (segment (start 44.9605 17.0305) (end 45.7325 17.0305) (width 1.5) (layer "B.Cu") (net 9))
 (segment (start 44.4475 17.0305) (end 45.7325 17.0305) (width 1.5) (layer "B.Cu") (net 9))
 (segment (start 45.7325 17.0305) (end 46.99 18.288) (width 1.5) (layer "B.Cu") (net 9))
 (segment (start 31.268 20.828) (end 31.268 21.59) (width 1.5) (layer "B.Cu") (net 11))
 (segment (start 33.7895 24.3815) (end 33.2715 24.3815) (width 1.5) (layer "B.Cu") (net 11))
 (segment (start 32.258 23.342) (end 31.268 22.352) (width 1.5) (layer "B.Cu") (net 11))
 (segment (start 33.2715 24.3815) (end 32.258 23.368) (width 1.5) (layer "B.Cu") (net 11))
 (segment (start 32.258 23.368) (end 32.258 23.342) (width 1.5) (layer "B.Cu") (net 11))
 (segment (start 32.0275 18.5395) (end 31.268 17.78) (width 1.5) (layer "B.Cu") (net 8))
 (segment (start 33.7895 18.5395) (end 32.0275 18.5395) (width 1.5) (layer "B.Cu") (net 8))
 (segment (start 31.2965 30.2235) (end 31.294 30.226) (width 1.5) (layer "B.Cu") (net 15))
 (segment (start 33.7895 30.2235) (end 31.2965 30.2235) (width 1.5) (layer "B.Cu") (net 15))
 (segment (start 33.7895 30.2235) (end 33.787 30.226) (width 1.5) (layer "B.Cu") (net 15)))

